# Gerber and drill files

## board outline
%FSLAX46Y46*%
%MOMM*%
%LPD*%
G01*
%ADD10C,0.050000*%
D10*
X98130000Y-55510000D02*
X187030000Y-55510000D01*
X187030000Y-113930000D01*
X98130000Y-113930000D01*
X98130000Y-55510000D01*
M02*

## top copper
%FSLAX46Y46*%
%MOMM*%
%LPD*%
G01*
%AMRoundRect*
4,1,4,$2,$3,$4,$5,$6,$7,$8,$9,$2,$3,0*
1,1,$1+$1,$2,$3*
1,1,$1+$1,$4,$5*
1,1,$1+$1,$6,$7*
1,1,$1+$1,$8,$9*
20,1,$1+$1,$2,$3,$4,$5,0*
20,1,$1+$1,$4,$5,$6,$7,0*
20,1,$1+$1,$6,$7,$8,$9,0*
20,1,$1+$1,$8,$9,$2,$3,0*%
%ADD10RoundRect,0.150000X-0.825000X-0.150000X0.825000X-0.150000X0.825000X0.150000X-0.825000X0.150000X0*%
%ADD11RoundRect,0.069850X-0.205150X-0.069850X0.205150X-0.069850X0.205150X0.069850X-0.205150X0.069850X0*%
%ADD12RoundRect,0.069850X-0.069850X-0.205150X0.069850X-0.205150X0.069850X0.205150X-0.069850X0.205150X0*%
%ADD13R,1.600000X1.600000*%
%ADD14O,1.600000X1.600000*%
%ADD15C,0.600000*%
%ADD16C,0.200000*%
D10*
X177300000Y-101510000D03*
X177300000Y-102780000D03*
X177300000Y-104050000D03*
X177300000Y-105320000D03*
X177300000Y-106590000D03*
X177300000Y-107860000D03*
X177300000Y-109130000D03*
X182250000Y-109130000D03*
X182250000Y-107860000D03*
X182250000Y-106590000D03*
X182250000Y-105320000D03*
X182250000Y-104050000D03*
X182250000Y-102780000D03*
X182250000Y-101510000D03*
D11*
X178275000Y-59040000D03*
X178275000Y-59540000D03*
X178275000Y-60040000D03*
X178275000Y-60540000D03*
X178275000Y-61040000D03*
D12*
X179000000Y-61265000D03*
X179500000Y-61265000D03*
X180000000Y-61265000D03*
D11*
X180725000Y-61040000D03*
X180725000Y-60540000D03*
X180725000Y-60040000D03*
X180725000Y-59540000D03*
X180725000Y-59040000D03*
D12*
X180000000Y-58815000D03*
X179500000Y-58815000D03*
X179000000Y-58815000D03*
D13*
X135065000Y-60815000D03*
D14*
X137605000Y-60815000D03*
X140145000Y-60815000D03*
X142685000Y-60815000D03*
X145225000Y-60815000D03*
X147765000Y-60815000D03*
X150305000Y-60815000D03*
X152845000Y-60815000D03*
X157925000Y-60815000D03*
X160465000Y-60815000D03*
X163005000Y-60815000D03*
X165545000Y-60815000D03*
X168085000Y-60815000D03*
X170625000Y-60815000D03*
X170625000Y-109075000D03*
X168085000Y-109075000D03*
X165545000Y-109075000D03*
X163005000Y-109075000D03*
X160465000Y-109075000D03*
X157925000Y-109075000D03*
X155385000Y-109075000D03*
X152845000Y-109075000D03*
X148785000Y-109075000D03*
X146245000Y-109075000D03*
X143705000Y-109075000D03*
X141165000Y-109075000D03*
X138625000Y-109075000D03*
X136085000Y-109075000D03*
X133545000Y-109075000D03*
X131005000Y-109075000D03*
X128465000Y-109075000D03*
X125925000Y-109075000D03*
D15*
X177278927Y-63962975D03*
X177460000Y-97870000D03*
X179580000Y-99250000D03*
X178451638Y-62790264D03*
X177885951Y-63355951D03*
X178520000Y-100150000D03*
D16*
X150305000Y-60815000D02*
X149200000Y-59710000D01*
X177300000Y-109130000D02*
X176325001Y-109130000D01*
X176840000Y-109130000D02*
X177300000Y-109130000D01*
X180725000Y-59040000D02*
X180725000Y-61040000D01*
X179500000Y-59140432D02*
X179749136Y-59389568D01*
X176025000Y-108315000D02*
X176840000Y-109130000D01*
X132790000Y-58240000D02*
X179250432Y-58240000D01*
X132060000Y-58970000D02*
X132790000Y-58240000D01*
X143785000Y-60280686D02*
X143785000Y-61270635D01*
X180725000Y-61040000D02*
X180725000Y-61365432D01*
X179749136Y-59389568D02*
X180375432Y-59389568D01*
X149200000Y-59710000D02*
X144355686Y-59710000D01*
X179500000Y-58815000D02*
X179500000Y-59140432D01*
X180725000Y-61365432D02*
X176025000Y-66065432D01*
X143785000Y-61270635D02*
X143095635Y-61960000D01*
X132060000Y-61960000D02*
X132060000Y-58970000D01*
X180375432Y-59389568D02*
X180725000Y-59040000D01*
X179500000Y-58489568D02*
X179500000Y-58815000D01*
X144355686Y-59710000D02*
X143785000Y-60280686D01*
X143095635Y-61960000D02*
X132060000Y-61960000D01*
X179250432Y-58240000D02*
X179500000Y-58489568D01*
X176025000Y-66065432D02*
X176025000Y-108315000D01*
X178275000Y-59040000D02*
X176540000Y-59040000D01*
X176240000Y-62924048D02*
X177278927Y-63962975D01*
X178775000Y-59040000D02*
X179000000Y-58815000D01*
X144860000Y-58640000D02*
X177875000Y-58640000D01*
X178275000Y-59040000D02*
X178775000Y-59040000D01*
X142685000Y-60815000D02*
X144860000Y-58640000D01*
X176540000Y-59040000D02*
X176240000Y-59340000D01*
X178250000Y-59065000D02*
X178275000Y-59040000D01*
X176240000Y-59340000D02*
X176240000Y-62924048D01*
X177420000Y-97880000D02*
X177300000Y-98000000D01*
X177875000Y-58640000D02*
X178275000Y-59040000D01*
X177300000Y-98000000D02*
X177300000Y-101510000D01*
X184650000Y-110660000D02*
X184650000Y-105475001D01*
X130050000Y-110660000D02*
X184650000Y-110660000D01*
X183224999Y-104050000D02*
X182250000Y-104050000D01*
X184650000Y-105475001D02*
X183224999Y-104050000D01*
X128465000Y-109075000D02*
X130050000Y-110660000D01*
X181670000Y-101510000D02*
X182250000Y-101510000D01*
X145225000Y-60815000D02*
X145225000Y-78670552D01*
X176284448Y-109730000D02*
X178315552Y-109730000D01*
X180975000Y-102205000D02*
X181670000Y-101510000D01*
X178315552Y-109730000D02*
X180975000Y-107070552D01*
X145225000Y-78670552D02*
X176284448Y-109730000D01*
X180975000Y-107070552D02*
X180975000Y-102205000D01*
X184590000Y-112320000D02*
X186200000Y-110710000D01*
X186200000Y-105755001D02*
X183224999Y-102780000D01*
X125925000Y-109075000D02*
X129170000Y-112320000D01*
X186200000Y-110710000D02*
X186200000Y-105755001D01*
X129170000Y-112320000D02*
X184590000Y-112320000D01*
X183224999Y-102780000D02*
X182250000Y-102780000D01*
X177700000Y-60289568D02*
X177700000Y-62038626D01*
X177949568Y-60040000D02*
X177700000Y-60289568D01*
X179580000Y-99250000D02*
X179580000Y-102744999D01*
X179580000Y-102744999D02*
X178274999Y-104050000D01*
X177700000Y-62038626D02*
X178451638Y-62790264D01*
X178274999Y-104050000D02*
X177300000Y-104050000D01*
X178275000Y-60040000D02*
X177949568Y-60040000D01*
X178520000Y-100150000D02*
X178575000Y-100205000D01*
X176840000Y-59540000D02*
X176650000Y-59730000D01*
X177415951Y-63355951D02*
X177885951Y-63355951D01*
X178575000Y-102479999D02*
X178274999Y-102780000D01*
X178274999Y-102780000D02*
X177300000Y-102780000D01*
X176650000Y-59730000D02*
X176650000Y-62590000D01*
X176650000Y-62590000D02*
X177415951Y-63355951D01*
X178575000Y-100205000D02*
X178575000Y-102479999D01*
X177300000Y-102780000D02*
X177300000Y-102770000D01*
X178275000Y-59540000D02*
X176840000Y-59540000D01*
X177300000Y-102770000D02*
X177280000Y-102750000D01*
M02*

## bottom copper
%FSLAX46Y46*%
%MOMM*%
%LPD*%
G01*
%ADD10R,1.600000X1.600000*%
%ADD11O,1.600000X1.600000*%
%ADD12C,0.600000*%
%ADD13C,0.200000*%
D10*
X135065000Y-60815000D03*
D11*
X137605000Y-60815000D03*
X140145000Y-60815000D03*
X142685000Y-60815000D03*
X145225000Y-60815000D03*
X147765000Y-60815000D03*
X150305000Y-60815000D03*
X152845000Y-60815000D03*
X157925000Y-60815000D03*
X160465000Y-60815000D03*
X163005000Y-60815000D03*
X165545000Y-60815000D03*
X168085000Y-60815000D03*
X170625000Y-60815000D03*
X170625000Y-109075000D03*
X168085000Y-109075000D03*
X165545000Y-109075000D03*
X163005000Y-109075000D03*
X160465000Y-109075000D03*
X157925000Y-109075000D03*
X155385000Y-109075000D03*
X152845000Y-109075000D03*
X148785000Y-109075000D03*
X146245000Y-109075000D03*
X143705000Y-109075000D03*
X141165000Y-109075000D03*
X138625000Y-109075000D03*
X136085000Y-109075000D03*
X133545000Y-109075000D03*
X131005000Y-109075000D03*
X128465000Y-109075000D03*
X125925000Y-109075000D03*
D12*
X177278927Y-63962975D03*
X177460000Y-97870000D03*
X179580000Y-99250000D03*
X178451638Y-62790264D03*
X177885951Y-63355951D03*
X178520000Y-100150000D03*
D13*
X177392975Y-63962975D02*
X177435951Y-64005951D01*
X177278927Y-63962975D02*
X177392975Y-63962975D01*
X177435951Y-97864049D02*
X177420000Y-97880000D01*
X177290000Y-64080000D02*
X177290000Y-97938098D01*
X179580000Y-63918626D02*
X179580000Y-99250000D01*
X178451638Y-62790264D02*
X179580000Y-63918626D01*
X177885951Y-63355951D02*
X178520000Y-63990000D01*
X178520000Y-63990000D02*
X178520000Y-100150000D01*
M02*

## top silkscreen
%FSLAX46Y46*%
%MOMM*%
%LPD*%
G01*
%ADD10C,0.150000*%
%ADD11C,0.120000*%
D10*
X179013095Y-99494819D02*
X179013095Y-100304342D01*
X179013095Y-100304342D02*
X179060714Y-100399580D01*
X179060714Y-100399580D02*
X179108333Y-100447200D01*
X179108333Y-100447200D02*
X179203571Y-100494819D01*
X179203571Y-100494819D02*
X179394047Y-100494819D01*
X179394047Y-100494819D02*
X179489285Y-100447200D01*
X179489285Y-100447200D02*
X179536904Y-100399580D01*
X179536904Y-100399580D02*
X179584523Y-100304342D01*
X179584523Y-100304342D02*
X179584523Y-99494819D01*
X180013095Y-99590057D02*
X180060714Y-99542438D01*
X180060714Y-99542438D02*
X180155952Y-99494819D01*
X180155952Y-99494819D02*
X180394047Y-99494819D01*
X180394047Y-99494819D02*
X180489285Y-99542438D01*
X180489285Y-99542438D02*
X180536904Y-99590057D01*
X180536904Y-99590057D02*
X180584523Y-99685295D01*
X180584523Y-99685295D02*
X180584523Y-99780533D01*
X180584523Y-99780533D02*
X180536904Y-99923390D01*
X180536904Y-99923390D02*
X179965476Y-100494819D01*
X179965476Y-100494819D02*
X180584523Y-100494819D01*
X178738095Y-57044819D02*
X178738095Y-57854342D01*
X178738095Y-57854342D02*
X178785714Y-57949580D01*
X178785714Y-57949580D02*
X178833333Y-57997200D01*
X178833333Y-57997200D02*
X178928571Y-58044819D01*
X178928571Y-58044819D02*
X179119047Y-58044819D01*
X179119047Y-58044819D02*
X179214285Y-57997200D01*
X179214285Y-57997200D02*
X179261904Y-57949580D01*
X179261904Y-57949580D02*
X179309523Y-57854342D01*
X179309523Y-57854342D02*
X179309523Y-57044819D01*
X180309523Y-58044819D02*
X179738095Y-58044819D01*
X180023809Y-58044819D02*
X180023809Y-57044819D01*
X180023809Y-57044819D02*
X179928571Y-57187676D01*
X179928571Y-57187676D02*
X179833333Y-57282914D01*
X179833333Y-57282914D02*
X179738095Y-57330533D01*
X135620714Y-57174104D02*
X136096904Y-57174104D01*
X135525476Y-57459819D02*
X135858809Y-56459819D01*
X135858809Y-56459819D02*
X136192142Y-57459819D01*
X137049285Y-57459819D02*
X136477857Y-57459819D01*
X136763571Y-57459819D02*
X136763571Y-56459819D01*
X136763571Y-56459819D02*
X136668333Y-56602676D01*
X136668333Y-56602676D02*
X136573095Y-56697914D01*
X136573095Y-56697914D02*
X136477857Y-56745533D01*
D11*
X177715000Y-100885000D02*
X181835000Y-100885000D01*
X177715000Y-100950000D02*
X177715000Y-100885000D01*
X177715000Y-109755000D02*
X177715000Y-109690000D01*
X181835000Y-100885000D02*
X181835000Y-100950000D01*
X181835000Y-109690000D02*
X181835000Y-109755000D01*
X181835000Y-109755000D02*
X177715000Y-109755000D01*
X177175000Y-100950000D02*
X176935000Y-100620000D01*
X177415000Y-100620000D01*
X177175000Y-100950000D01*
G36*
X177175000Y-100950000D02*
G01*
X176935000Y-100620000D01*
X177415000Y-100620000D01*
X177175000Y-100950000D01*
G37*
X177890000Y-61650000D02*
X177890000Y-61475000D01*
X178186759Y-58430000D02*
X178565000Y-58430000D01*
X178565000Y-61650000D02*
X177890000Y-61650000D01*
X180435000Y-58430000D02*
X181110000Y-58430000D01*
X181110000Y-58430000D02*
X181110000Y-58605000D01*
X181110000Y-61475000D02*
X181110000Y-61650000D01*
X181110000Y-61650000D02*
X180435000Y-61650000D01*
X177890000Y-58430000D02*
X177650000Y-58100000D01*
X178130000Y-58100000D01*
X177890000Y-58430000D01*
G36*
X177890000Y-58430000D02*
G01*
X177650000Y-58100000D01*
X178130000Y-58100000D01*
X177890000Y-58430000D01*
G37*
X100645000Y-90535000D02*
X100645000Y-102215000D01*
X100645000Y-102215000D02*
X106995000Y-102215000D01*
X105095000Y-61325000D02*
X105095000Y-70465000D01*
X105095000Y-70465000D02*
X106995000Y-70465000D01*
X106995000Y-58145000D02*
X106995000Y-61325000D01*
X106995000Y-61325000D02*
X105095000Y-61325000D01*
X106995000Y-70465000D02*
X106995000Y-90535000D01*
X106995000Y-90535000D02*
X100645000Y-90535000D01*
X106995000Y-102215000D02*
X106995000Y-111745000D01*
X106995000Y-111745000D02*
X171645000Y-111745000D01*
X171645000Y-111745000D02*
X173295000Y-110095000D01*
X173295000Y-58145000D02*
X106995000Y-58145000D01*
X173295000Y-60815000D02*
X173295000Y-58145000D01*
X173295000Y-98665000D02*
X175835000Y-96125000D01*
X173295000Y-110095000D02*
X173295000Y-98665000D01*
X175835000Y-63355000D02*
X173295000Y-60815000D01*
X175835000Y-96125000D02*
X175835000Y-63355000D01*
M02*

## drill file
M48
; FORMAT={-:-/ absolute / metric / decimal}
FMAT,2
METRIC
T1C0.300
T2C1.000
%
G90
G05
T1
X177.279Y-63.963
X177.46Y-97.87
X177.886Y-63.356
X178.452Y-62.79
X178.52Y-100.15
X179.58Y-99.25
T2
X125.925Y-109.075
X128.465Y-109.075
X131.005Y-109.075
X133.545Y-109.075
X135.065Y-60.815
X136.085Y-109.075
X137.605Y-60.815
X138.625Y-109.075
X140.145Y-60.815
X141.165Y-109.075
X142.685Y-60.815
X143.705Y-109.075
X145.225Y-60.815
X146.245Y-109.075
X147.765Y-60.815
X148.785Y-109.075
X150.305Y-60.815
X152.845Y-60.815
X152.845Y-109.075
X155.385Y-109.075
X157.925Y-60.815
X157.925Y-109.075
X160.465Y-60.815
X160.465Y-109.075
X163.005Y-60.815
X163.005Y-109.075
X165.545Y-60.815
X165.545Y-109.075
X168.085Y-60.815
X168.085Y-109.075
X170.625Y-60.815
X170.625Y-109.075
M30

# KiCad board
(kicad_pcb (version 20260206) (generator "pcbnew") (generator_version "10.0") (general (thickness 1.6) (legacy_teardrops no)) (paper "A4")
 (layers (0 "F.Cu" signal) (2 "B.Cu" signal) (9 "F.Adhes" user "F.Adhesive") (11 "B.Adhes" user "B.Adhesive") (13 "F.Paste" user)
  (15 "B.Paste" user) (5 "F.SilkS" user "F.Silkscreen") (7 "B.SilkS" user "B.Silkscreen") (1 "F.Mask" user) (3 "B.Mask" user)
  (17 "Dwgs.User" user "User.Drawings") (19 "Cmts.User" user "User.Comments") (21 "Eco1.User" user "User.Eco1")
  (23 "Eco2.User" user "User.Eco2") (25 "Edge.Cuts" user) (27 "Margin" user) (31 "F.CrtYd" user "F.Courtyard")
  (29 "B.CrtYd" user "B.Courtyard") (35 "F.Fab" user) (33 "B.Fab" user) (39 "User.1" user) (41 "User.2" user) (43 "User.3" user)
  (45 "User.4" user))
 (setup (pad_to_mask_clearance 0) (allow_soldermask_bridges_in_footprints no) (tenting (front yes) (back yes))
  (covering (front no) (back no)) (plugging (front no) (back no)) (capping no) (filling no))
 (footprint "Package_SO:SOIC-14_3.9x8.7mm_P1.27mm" (layer "F.Cu") (at 179.775 105.32)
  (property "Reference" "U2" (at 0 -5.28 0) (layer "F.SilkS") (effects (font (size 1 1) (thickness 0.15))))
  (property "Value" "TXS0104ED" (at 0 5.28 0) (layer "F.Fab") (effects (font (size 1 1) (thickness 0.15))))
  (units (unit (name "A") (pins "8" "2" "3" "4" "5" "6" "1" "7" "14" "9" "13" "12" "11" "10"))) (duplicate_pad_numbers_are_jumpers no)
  (fp_line (start -2.06 -4.435) (end 2.06 -4.435) (stroke (width 0.12) (type solid)) (layer "F.SilkS"))
  (fp_line (start -2.06 -4.37) (end -2.06 -4.435) (stroke (width 0.12) (type solid)) (layer "F.SilkS"))
  (fp_line (start -2.06 4.435) (end -2.06 4.37) (stroke (width 0.12) (type solid)) (layer "F.SilkS"))
  (fp_line (start 2.06 -4.435) (end 2.06 -4.37) (stroke (width 0.12) (type solid)) (layer "F.SilkS"))
  (fp_line (start 2.06 4.37) (end 2.06 4.435) (stroke (width 0.12) (type solid)) (layer "F.SilkS"))
  (fp_line (start 2.06 4.435) (end -2.06 4.435) (stroke (width 0.12) (type solid)) (layer "F.SilkS"))
  (fp_poly (pts (xy -2.6 -4.37) (xy -2.84 -4.7) (xy -2.36 -4.7)) (stroke (width 0.12) (type solid)) (fill yes) (layer "F.SilkS"))
  (pad "1" smd roundrect (at -2.475 -3.81) (size 1.95 0.6) (layers "F.Cu" "F.Mask" "F.Paste") (roundrect_rratio 0.25) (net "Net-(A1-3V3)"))
  (pad "2" smd roundrect (at -2.475 -2.54) (size 1.95 0.6) (layers "F.Cu" "F.Mask" "F.Paste") (roundrect_rratio 0.25)
   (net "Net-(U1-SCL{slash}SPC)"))
  (pad "3" smd roundrect (at -2.475 -1.27) (size 1.95 0.6) (layers "F.Cu" "F.Mask" "F.Paste") (roundrect_rratio 0.25)
   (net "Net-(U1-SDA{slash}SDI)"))
  (pad "4" smd roundrect (at -2.475 0) (size 1.95 0.6) (layers "F.Cu" "F.Mask" "F.Paste") (roundrect_rratio 0.25)
   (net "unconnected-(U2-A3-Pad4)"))
  (pad "5" smd roundrect (at -2.475 1.27) (size 1.95 0.6) (layers "F.Cu" "F.Mask" "F.Paste") (roundrect_rratio 0.25)
   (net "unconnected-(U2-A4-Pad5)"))
  (pad "6" smd roundrect (at -2.475 2.54) (size 1.95 0.6) (layers "F.Cu" "F.Mask" "F.Paste") (roundrect_rratio 0.25)
   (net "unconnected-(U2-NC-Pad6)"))
  (pad "7" smd roundrect (at -2.475 3.81) (size 1.95 0.6) (layers "F.Cu" "F.Mask" "F.Paste") (roundrect_rratio 0.25) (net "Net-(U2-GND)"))
  (pad "8" smd roundrect (at 2.475 3.81) (size 1.95 0.6) (layers "F.Cu" "F.Mask" "F.Paste") (roundrect_rratio 0.25)
   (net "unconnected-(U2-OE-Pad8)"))
  (pad "9" smd roundrect (at 2.475 2.54) (size 1.95 0.6) (layers "F.Cu" "F.Mask" "F.Paste") (roundrect_rratio 0.25)
   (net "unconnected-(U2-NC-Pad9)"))
  (pad "10" smd roundrect (at 2.475 1.27) (size 1.95 0.6) (layers "F.Cu" "F.Mask" "F.Paste") (roundrect_rratio 0.25)
   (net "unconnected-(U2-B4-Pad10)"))
  (pad "11" smd roundrect (at 2.475 0) (size 1.95 0.6) (layers "F.Cu" "F.Mask" "F.Paste") (roundrect_rratio 0.25)
   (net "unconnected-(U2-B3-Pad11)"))
  (pad "12" smd roundrect (at 2.475 -1.27) (size 1.95 0.6) (layers "F.Cu" "F.Mask" "F.Paste") (roundrect_rratio 0.25)
   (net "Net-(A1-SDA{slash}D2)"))
  (pad "13" smd roundrect (at 2.475 -2.54) (size 1.95 0.6) (layers "F.Cu" "F.Mask" "F.Paste") (roundrect_rratio 0.25)
   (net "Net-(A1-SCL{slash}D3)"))
  (pad "14" smd roundrect (at 2.475 -3.81) (size 1.95 0.6) (layers "F.Cu" "F.Mask" "F.Paste") (roundrect_rratio 0.25) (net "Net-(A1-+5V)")))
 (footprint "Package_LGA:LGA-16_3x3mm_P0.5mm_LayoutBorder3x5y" (layer "F.Cu") (at 179.5 60.04)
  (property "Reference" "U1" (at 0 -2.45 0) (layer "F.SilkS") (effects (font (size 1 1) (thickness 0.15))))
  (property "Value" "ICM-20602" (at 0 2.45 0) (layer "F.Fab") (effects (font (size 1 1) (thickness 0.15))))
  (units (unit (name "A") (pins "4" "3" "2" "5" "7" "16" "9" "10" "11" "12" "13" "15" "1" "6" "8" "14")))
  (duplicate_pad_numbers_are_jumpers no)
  (fp_line (start -1.61 1.61) (end -1.61 1.435) (stroke (width 0.12) (type solid)) (layer "F.SilkS"))
  (fp_line (start -1.313241 -1.61) (end -0.935 -1.61) (stroke (width 0.12) (type solid)) (layer "F.SilkS"))
  (fp_line (start -0.935 1.61) (end -1.61 1.61) (stroke (width 0.12) (type solid)) (layer "F.SilkS"))
  (fp_line (start 0.935 -1.61) (end 1.61 -1.61) (stroke (width 0.12) (type solid)) (layer "F.SilkS"))
  (fp_line (start 1.61 -1.61) (end 1.61 -1.435) (stroke (width 0.12) (type solid)) (layer "F.SilkS"))
  (fp_line (start 1.61 1.435) (end 1.61 1.61) (stroke (width 0.12) (type solid)) (layer "F.SilkS"))
  (fp_line (start 1.61 1.61) (end 0.935 1.61) (stroke (width 0.12) (type solid)) (layer "F.SilkS"))
  (fp_poly (pts (xy -1.61 -1.61) (xy -1.85 -1.94) (xy -1.37 -1.94)) (stroke (width 0.12) (type solid)) (fill yes) (layer "F.SilkS"))
  (pad "1" smd roundrect (at -1.225 -1) (size 0.55 0.2794) (layers "F.Cu" "F.Mask" "F.Paste") (roundrect_rratio 0.25) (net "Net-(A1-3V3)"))
  (pad "2" smd roundrect (at -1.225 -0.5) (size 0.55 0.2794) (layers "F.Cu" "F.Mask" "F.Paste") (roundrect_rratio 0.25)
   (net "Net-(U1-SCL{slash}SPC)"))
  (pad "3" smd roundrect (at -1.225 0) (size 0.55 0.2794) (layers "F.Cu" "F.Mask" "F.Paste") (roundrect_rratio 0.25)
   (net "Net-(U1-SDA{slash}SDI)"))
  (pad "4" smd roundrect (at -1.225 0.5) (size 0.55 0.2794) (layers "F.Cu" "F.Mask" "F.Paste") (roundrect_rratio 0.25)
   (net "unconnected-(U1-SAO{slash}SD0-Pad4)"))
  (pad "5" smd roundrect (at -1.225 1) (size 0.55 0.2794) (layers "F.Cu" "F.Mask" "F.Paste") (roundrect_rratio 0.25)
   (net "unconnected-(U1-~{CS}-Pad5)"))
  (pad "6" smd roundrect (at -0.5 1.225) (size 0.2794 0.55) (layers "F.Cu" "F.Mask" "F.Paste") (roundrect_rratio 0.25)
   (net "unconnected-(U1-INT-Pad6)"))
  (pad "7" smd roundrect (at 0 1.225) (size 0.2794 0.55) (layers "F.Cu" "F.Mask" "F.Paste") (roundrect_rratio 0.25)
   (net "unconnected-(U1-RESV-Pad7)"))
  (pad "8" smd roundrect (at 0.5 1.225) (size 0.2794 0.55) (layers "F.Cu" "F.Mask" "F.Paste") (roundrect_rratio 0.25)
   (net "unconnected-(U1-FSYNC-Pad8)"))
  (pad "9" smd roundrect (at 1.225 1) (size 0.55 0.2794) (layers "F.Cu" "F.Mask" "F.Paste") (roundrect_rratio 0.25) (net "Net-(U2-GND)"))
  (pad "10" smd roundrect (at 1.225 0.5) (size 0.55 0.2794) (layers "F.Cu" "F.Mask" "F.Paste") (roundrect_rratio 0.25) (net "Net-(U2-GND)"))
  (pad "11" smd roundrect (at 1.225 0) (size 0.55 0.2794) (layers "F.Cu" "F.Mask" "F.Paste") (roundrect_rratio 0.25) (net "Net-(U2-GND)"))
  (pad "12" smd roundrect (at 1.225 -0.5) (size 0.55 0.2794) (layers "F.Cu" "F.Mask" "F.Paste") (roundrect_rratio 0.25) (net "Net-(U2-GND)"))
  (pad "13" smd roundrect (at 1.225 -1) (size 0.55 0.2794) (layers "F.Cu" "F.Mask" "F.Paste") (roundrect_rratio 0.25) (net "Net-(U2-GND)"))
  (pad "14" smd roundrect (at 0.5 -1.225) (size 0.2794 0.55) (layers "F.Cu" "F.Mask" "F.Paste") (roundrect_rratio 0.25)
   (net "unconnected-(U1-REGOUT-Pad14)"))
  (pad "15" smd roundrect (at 0 -1.225) (size 0.2794 0.55) (layers "F.Cu" "F.Mask" "F.Paste") (roundrect_rratio 0.25) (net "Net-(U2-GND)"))
  (pad "16" smd roundrect (at -0.5 -1.225) (size 0.2794 0.55) (layers "F.Cu" "F.Mask" "F.Paste") (roundrect_rratio 0.25)
   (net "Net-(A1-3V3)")))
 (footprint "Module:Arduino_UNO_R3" (layer "F.Cu") (at 135.065 60.815)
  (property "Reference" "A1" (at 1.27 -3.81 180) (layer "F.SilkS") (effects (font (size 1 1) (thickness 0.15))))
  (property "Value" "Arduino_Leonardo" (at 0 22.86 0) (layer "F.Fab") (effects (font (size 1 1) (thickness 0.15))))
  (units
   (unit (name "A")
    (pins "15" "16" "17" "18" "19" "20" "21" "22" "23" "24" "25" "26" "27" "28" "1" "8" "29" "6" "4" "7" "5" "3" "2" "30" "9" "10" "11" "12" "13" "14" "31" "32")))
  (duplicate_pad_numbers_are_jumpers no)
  (fp_line (start -34.42 29.72) (end -34.42 41.4) (stroke (width 0.12) (type solid)) (layer "F.SilkS"))
  (fp_line (start -34.42 41.4) (end -28.07 41.4) (stroke (width 0.12) (type solid)) (layer "F.SilkS"))
  (fp_line (start -29.97 0.51) (end -29.97 9.65) (stroke (width 0.12) (type solid)) (layer "F.SilkS"))
  (fp_line (start -29.97 9.65) (end -28.07 9.65) (stroke (width 0.12) (type solid)) (layer "F.SilkS"))
  (fp_line (start -28.07 -2.67) (end -28.07 0.51) (stroke (width 0.12) (type solid)) (layer "F.SilkS"))
  (fp_line (start -28.07 0.51) (end -29.97 0.51) (stroke (width 0.12) (type solid)) (layer "F.SilkS"))
  (fp_line (start -28.07 9.65) (end -28.07 29.72) (stroke (width 0.12) (type solid)) (layer "F.SilkS"))
  (fp_line (start -28.07 29.72) (end -34.42 29.72) (stroke (width 0.12) (type solid)) (layer "F.SilkS"))
  (fp_line (start -28.07 41.4) (end -28.07 50.93) (stroke (width 0.12) (type solid)) (layer "F.SilkS"))
  (fp_line (start -28.07 50.93) (end 36.58 50.93) (stroke (width 0.12) (type solid)) (layer "F.SilkS"))
  (fp_line (start 36.58 50.93) (end 38.23 49.28) (stroke (width 0.12) (type solid)) (layer "F.SilkS"))
  (fp_line (start 38.23 -2.67) (end -28.07 -2.67) (stroke (width 0.12) (type solid)) (layer "F.SilkS"))
  (fp_line (start 38.23 0) (end 38.23 -2.67) (stroke (width 0.12) (type solid)) (layer "F.SilkS"))
  (fp_line (start 38.23 37.85) (end 40.77 35.31) (stroke (width 0.12) (type solid)) (layer "F.SilkS"))
  (fp_line (start 38.23 49.28) (end 38.23 37.85) (stroke (width 0.12) (type solid)) (layer "F.SilkS"))
  (fp_line (start 40.77 2.54) (end 38.23 0) (stroke (width 0.12) (type solid)) (layer "F.SilkS"))
  (fp_line (start 40.77 35.31) (end 40.77 2.54) (stroke (width 0.12) (type solid)) (layer "F.SilkS"))
  (pad "1" thru_hole rect (at 0 0 90) (size 1.6 1.6) (drill 1) (layers "*.Cu" "*.Mask") (remove_unused_layers no)
   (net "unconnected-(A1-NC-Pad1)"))
  (pad "2" thru_hole oval (at 2.54 0 90) (size 1.6 1.6) (drill 1) (layers "*.Cu" "*.Mask") (remove_unused_layers no)
   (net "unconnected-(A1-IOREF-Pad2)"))
  (pad "3" thru_hole oval (at 5.08 0 90) (size 1.6 1.6) (drill 1) (layers "*.Cu" "*.Mask") (remove_unused_layers no)
   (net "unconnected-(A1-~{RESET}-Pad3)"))
  (pad "4" thru_hole oval (at 7.62 0 90) (size 1.6 1.6) (drill 1) (layers "*.Cu" "*.Mask") (remove_unused_layers no) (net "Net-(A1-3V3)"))
  (pad "5" thru_hole oval (at 10.16 0 90) (size 1.6 1.6) (drill 1) (layers "*.Cu" "*.Mask") (remove_unused_layers no) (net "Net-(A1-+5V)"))
  (pad "6" thru_hole oval (at 12.7 0 90) (size 1.6 1.6) (drill 1) (layers "*.Cu" "*.Mask") (remove_unused_layers no)
   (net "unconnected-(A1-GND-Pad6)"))
  (pad "7" thru_hole oval (at 15.24 0 90) (size 1.6 1.6) (drill 1) (layers "*.Cu" "*.Mask") (remove_unused_layers no) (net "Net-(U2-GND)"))
  (pad "8" thru_hole oval (at 17.78 0 90) (size 1.6 1.6) (drill 1) (layers "*.Cu" "*.Mask") (remove_unused_layers no)
   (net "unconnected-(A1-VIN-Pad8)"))
  (pad "9" thru_hole oval (at 22.86 0 90) (size 1.6 1.6) (drill 1) (layers "*.Cu" "*.Mask") (remove_unused_layers no)
   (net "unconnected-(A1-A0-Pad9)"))
  (pad "10" thru_hole oval (at 25.4 0 90) (size 1.6 1.6) (drill 1) (layers "*.Cu" "*.Mask") (remove_unused_layers no)
   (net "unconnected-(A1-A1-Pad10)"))
  (pad "11" thru_hole oval (at 27.94 0 90) (size 1.6 1.6) (drill 1) (layers "*.Cu" "*.Mask") (remove_unused_layers no)
   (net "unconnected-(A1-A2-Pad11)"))
  (pad "12" thru_hole oval (at 30.48 0 90) (size 1.6 1.6) (drill 1) (layers "*.Cu" "*.Mask") (remove_unused_layers no)
   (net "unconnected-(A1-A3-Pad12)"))
  (pad "13" thru_hole oval (at 33.02 0 90) (size 1.6 1.6) (drill 1) (layers "*.Cu" "*.Mask") (remove_unused_layers no)
   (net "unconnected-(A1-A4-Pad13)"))
  (pad "14" thru_hole oval (at 35.56 0 90) (size 1.6 1.6) (drill 1) (layers "*.Cu" "*.Mask") (remove_unused_layers no)
   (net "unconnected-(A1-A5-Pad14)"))
  (pad "15" thru_hole oval (at 35.56 48.26 90) (size 1.6 1.6) (drill 1) (layers "*.Cu" "*.Mask") (remove_unused_layers no)
   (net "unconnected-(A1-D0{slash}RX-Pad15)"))
  (pad "16" thru_hole oval (at 33.02 48.26 90) (size 1.6 1.6) (drill 1) (layers "*.Cu" "*.Mask") (remove_unused_layers no)
   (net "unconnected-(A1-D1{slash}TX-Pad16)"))
  (pad "17" thru_hole oval (at 30.48 48.26 90) (size 1.6 1.6) (drill 1) (layers "*.Cu" "*.Mask") (remove_unused_layers no)
   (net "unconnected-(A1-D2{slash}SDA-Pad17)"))
  (pad "18" thru_hole oval (at 27.94 48.26 90) (size 1.6 1.6) (drill 1) (layers "*.Cu" "*.Mask") (remove_unused_layers no)
   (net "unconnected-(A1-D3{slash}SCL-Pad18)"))
  (pad "19" thru_hole oval (at 25.4 48.26 90) (size 1.6 1.6) (drill 1) (layers "*.Cu" "*.Mask") (remove_unused_layers no)
   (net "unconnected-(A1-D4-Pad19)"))
  (pad "20" thru_hole oval (at 22.86 48.26 90) (size 1.6 1.6) (drill 1) (layers "*.Cu" "*.Mask") (remove_unused_layers no)
   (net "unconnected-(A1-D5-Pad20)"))
  (pad "21" thru_hole oval (at 20.32 48.26 90) (size 1.6 1.6) (drill 1) (layers "*.Cu" "*.Mask") (remove_unused_layers no)
   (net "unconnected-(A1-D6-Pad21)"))
  (pad "22" thru_hole oval (at 17.78 48.26 90) (size 1.6 1.6) (drill 1) (layers "*.Cu" "*.Mask") (remove_unused_layers no)
   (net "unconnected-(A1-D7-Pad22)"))
  (pad "23" thru_hole oval (at 13.72 48.26 90) (size 1.6 1.6) (drill 1) (layers "*.Cu" "*.Mask") (remove_unused_layers no)
   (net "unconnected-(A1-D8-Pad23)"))
  (pad "24" thru_hole oval (at 11.18 48.26 90) (size 1.6 1.6) (drill 1) (layers "*.Cu" "*.Mask") (remove_unused_layers no)
   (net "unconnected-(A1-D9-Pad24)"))
  (pad "25" thru_hole oval (at 8.64 48.26 90) (size 1.6 1.6) (drill 1) (layers "*.Cu" "*.Mask") (remove_unused_layers no)
   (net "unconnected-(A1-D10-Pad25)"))
  (pad "26" thru_hole oval (at 6.1 48.26 90) (size 1.6 1.6) (drill 1) (layers "*.Cu" "*.Mask") (remove_unused_layers no)
   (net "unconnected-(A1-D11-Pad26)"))
  (pad "27" thru_hole oval (at 3.56 48.26 90) (size 1.6 1.6) (drill 1) (layers "*.Cu" "*.Mask") (remove_unused_layers no)
   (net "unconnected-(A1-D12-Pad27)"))
  (pad "28" thru_hole oval (at 1.02 48.26 90) (size 1.6 1.6) (drill 1) (layers "*.Cu" "*.Mask") (remove_unused_layers no)
   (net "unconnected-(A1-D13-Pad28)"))
  (pad "29" thru_hole oval (at -1.52 48.26 90) (size 1.6 1.6) (drill 1) (layers "*.Cu" "*.Mask") (remove_unused_layers no)
   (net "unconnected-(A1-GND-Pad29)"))
  (pad "30" thru_hole oval (at -4.06 48.26 90) (size 1.6 1.6) (drill 1) (layers "*.Cu" "*.Mask") (remove_unused_layers no)
   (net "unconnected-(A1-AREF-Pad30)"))
  (pad "31" thru_hole oval (at -6.6 48.26 90) (size 1.6 1.6) (drill 1) (layers "*.Cu" "*.Mask") (remove_unused_layers no)
   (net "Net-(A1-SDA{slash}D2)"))
  (pad "32" thru_hole oval (at -9.14 48.26 90) (size 1.6 1.6) (drill 1) (layers "*.Cu" "*.Mask") (remove_unused_layers no)
   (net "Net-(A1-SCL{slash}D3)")))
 (gr_rect (start 98.13 55.51) (end 187.03 113.93) (stroke (width 0.05) (type solid)) (fill no) (layer "Edge.Cuts"))
 (segment (start 150.305 60.815) (end 149.2 59.71) (width 0.2) (layer "F.Cu") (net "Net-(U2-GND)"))
 (segment (start 177.3 109.13) (end 176.325001 109.13) (width 0.2) (layer "F.Cu") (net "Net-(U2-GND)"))
 (segment (start 176.84 109.13) (end 177.3 109.13) (width 0.2) (layer "F.Cu") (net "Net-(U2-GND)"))
 (segment (start 180.725 59.04) (end 180.725 61.04) (width 0.2) (layer "F.Cu") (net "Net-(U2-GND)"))
 (segment (start 179.5 59.140432) (end 179.749136 59.389568) (width 0.2) (layer "F.Cu") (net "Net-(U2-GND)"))
 (segment (start 176.025 108.315) (end 176.84 109.13) (width 0.2) (layer "F.Cu") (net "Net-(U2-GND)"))
 (segment (start 132.79 58.24) (end 179.250432 58.24) (width 0.2) (layer "F.Cu") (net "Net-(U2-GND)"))
 (segment (start 132.06 58.97) (end 132.79 58.24) (width 0.2) (layer "F.Cu") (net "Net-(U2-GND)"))
 (segment (start 143.785 60.280686) (end 143.785 61.270635) (width 0.2) (layer "F.Cu") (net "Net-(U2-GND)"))
 (segment (start 180.725 61.04) (end 180.725 61.365432) (width 0.2) (layer "F.Cu") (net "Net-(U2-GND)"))
 (segment (start 179.749136 59.389568) (end 180.375432 59.389568) (width 0.2) (layer "F.Cu") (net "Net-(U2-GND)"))
 (segment (start 149.2 59.71) (end 144.355686 59.71) (width 0.2) (layer "F.Cu") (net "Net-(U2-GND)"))
 (segment (start 179.5 58.815) (end 179.5 59.140432) (width 0.2) (layer "F.Cu") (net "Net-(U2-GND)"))
 (segment (start 180.725 61.365432) (end 176.025 66.065432) (width 0.2) (layer "F.Cu") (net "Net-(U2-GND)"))
 (segment (start 143.785 61.270635) (end 143.095635 61.96) (width 0.2) (layer "F.Cu") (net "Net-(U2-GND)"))
 (segment (start 132.06 61.96) (end 132.06 58.97) (width 0.2) (layer "F.Cu") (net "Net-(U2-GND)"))
 (segment (start 180.375432 59.389568) (end 180.725 59.04) (width 0.2) (layer "F.Cu") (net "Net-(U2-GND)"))
 (segment (start 179.5 58.489568) (end 179.5 58.815) (width 0.2) (layer "F.Cu") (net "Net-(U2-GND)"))
 (segment (start 144.355686 59.71) (end 143.785 60.280686) (width 0.2) (layer "F.Cu") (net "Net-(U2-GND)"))
 (segment (start 143.095635 61.96) (end 132.06 61.96) (width 0.2) (layer "F.Cu") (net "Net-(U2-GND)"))
 (segment (start 179.250432 58.24) (end 179.5 58.489568) (width 0.2) (layer "F.Cu") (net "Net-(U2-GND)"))
 (segment (start 176.025 66.065432) (end 176.025 108.315) (width 0.2) (layer "F.Cu") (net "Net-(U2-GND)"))
 (segment (start 178.275 59.04) (end 176.54 59.04) (width 0.2) (layer "F.Cu") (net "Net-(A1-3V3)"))
 (segment (start 176.24 62.924048) (end 177.278927 63.962975) (width 0.2) (layer "F.Cu") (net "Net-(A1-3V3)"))
 (segment (start 178.775 59.04) (end 179 58.815) (width 0.2) (layer "F.Cu") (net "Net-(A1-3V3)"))
 (segment (start 144.86 58.64) (end 177.875 58.64) (width 0.2) (layer "F.Cu") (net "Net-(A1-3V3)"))
 (segment (start 178.275 59.04) (end 178.775 59.04) (width 0.2) (layer "F.Cu") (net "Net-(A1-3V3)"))
 (segment (start 142.685 60.815) (end 144.86 58.64) (width 0.2) (layer "F.Cu") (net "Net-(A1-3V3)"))
 (segment (start 176.54 59.04) (end 176.24 59.34) (width 0.2) (layer "F.Cu") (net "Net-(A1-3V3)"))
 (segment (start 178.25 59.065) (end 178.275 59.04) (width 0.2) (layer "F.Cu") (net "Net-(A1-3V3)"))
 (segment (start 176.24 59.34) (end 176.24 62.924048) (width 0.2) (layer "F.Cu") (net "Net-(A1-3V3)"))
 (segment (start 177.42 97.88) (end 177.3 98) (width 0.2) (layer "F.Cu") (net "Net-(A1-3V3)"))
 (segment (start 177.875 58.64) (end 178.275 59.04) (width 0.2) (layer "F.Cu") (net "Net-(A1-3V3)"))
 (segment (start 177.3 98) (end 177.3 101.51) (width 0.2) (layer "F.Cu") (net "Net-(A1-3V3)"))
 (via (at 177.278927 63.962975) (size 0.6) (drill 0.3) (layers "F.Cu" "B.Cu") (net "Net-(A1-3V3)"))
 (via (at 177.46 97.87) (size 0.6) (drill 0.3) (layers "F.Cu" "B.Cu") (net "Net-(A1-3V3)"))
 (segment (start 177.392975 63.962975) (end 177.435951 64.005951) (width 0.2) (layer "B.Cu") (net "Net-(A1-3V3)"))
 (segment (start 177.278927 63.962975) (end 177.392975 63.962975) (width 0.2) (layer "B.Cu") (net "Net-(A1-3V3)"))
 (segment (start 177.435951 97.864049) (end 177.42 97.88) (width 0.2) (layer "B.Cu") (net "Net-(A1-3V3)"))
 (segment (start 177.29 64.08) (end 177.29 97.938098) (width 0.2) (layer "B.Cu") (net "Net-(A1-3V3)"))
 (segment (start 184.65 110.66) (end 184.65 105.475001) (width 0.2) (layer "F.Cu") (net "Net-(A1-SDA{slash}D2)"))
 (segment (start 130.05 110.66) (end 184.65 110.66) (width 0.2) (layer "F.Cu") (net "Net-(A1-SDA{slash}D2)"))
 (segment (start 183.224999 104.05) (end 182.25 104.05) (width 0.2) (layer "F.Cu") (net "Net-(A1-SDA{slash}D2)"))
 (segment (start 184.65 105.475001) (end 183.224999 104.05) (width 0.2) (layer "F.Cu") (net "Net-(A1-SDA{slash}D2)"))
 (segment (start 128.465 109.075) (end 130.05 110.66) (width 0.2) (layer "F.Cu") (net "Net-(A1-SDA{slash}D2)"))
 (segment (start 181.67 101.51) (end 182.25 101.51) (width 0.2) (layer "F.Cu") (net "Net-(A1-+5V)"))
 (segment (start 145.225 60.815) (end 145.225 78.670552) (width 0.2) (layer "F.Cu") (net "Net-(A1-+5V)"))
 (segment (start 176.284448 109.73) (end 178.315552 109.73) (width 0.2) (layer "F.Cu") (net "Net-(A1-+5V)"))
 (segment (start 180.975 102.205) (end 181.67 101.51) (width 0.2) (layer "F.Cu") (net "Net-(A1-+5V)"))
 (segment (start 178.315552 109.73) (end 180.975 107.070552) (width 0.2) (layer "F.Cu") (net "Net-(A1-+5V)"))
 (segment (start 145.225 78.670552) (end 176.284448 109.73) (width 0.2) (layer "F.Cu") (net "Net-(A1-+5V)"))
 (segment (start 180.975 107.070552) (end 180.975 102.205) (width 0.2) (layer "F.Cu") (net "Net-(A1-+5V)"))
 (segment (start 184.59 112.32) (end 186.2 110.71) (width 0.2) (layer "F.Cu") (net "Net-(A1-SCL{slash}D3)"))
 (segment (start 186.2 105.755001) (end 183.224999 102.78) (width 0.2) (layer "F.Cu") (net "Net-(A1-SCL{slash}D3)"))
 (segment (start 125.925 109.075) (end 129.17 112.32) (width 0.2) (layer "F.Cu") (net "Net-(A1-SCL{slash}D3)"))
 (segment (start 186.2 110.71) (end 186.2 105.755001) (width 0.2) (layer "F.Cu") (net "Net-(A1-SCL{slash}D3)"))
 (segment (start 129.17 112.32) (end 184.59 112.32) (width 0.2) (layer "F.Cu") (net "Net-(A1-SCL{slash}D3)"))
 (segment (start 183.224999 102.78) (end 182.25 102.78) (width 0.2) (layer "F.Cu") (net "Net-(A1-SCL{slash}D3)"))
 (segment (start 177.7 60.289568) (end 177.7 62.038626) (width 0.2) (layer "F.Cu") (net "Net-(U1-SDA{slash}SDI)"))
 (segment (start 177.949568 60.04) (end 177.7 60.289568) (width 0.2) (layer "F.Cu") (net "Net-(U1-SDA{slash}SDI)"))
 (segment (start 179.58 99.25) (end 179.58 102.744999) (width 0.2) (layer "F.Cu") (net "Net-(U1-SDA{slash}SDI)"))
 (segment (start 179.58 102.744999) (end 178.274999 104.05) (width 0.2) (layer "F.Cu") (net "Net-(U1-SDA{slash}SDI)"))
 (segment (start 177.7 62.038626) (end 178.451638 62.790264) (width 0.2) (layer "F.Cu") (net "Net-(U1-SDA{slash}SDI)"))
 (segment (start 178.274999 104.05) (end 177.3 104.05) (width 0.2) (layer "F.Cu") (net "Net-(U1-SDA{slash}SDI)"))
 (segment (start 178.275 60.04) (end 177.949568 60.04) (width 0.2) (layer "F.Cu") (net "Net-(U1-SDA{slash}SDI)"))
 (via (at 179.58 99.25) (size 0.6) (drill 0.3) (layers "F.Cu" "B.Cu") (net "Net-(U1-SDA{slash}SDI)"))
 (via (at 178.451638 62.790264) (size 0.6) (drill 0.3) (layers "F.Cu" "B.Cu") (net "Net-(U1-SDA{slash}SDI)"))
 (segment (start 179.58 63.918626) (end 179.58 99.25) (width 0.2) (layer "B.Cu") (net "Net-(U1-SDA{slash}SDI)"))
 (segment (start 178.451638 62.790264) (end 179.58 63.918626) (width 0.2) (layer "B.Cu") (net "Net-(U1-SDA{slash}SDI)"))
 (segment (start 178.52 100.15) (end 178.575 100.205) (width 0.2) (layer "F.Cu") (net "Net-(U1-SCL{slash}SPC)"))
 (segment (start 176.84 59.54) (end 176.65 59.73) (width 0.2) (layer "F.Cu") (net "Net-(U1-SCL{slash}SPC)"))
 (segment (start 177.415951 63.355951) (end 177.885951 63.355951) (width 0.2) (layer "F.Cu") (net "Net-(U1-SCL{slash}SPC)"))
 (segment (start 178.575 102.479999) (end 178.274999 102.78) (width 0.2) (layer "F.Cu") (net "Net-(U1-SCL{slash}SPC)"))
 (segment (start 178.274999 102.78) (end 177.3 102.78) (width 0.2) (layer "F.Cu") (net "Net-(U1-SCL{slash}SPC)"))
 (segment (start 176.65 59.73) (end 176.65 62.59) (width 0.2) (layer "F.Cu") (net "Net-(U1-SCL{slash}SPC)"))
 (segment (start 176.65 62.59) (end 177.415951 63.355951) (width 0.2) (layer "F.Cu") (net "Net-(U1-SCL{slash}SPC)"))
 (segment (start 178.575 100.205) (end 178.575 102.479999) (width 0.2) (layer "F.Cu") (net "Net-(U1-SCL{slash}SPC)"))
 (segment (start 177.3 102.78) (end 177.3 102.77) (width 0.2) (layer "F.Cu") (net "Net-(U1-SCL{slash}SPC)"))
 (segment (start 178.275 59.54) (end 176.84 59.54) (width 0.2) (layer "F.Cu") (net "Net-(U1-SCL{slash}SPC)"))
 (segment (start 177.3 102.77) (end 177.28 102.75) (width 0.2) (layer "F.Cu") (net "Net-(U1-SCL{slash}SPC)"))
 (via (at 177.885951 63.355951) (size 0.6) (drill 0.3) (layers "F.Cu" "B.Cu") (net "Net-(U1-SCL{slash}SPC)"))
 (via (at 178.52 100.15) (size 0.6) (drill 0.3) (layers "F.Cu" "B.Cu") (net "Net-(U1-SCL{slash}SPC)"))
 (segment (start 177.885951 63.355951) (end 178.52 63.99) (width 0.2) (layer "B.Cu") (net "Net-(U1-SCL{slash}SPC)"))
 (segment (start 178.52 63.99) (end 178.52 100.15) (width 0.2) (layer "B.Cu") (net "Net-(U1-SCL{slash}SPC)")))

